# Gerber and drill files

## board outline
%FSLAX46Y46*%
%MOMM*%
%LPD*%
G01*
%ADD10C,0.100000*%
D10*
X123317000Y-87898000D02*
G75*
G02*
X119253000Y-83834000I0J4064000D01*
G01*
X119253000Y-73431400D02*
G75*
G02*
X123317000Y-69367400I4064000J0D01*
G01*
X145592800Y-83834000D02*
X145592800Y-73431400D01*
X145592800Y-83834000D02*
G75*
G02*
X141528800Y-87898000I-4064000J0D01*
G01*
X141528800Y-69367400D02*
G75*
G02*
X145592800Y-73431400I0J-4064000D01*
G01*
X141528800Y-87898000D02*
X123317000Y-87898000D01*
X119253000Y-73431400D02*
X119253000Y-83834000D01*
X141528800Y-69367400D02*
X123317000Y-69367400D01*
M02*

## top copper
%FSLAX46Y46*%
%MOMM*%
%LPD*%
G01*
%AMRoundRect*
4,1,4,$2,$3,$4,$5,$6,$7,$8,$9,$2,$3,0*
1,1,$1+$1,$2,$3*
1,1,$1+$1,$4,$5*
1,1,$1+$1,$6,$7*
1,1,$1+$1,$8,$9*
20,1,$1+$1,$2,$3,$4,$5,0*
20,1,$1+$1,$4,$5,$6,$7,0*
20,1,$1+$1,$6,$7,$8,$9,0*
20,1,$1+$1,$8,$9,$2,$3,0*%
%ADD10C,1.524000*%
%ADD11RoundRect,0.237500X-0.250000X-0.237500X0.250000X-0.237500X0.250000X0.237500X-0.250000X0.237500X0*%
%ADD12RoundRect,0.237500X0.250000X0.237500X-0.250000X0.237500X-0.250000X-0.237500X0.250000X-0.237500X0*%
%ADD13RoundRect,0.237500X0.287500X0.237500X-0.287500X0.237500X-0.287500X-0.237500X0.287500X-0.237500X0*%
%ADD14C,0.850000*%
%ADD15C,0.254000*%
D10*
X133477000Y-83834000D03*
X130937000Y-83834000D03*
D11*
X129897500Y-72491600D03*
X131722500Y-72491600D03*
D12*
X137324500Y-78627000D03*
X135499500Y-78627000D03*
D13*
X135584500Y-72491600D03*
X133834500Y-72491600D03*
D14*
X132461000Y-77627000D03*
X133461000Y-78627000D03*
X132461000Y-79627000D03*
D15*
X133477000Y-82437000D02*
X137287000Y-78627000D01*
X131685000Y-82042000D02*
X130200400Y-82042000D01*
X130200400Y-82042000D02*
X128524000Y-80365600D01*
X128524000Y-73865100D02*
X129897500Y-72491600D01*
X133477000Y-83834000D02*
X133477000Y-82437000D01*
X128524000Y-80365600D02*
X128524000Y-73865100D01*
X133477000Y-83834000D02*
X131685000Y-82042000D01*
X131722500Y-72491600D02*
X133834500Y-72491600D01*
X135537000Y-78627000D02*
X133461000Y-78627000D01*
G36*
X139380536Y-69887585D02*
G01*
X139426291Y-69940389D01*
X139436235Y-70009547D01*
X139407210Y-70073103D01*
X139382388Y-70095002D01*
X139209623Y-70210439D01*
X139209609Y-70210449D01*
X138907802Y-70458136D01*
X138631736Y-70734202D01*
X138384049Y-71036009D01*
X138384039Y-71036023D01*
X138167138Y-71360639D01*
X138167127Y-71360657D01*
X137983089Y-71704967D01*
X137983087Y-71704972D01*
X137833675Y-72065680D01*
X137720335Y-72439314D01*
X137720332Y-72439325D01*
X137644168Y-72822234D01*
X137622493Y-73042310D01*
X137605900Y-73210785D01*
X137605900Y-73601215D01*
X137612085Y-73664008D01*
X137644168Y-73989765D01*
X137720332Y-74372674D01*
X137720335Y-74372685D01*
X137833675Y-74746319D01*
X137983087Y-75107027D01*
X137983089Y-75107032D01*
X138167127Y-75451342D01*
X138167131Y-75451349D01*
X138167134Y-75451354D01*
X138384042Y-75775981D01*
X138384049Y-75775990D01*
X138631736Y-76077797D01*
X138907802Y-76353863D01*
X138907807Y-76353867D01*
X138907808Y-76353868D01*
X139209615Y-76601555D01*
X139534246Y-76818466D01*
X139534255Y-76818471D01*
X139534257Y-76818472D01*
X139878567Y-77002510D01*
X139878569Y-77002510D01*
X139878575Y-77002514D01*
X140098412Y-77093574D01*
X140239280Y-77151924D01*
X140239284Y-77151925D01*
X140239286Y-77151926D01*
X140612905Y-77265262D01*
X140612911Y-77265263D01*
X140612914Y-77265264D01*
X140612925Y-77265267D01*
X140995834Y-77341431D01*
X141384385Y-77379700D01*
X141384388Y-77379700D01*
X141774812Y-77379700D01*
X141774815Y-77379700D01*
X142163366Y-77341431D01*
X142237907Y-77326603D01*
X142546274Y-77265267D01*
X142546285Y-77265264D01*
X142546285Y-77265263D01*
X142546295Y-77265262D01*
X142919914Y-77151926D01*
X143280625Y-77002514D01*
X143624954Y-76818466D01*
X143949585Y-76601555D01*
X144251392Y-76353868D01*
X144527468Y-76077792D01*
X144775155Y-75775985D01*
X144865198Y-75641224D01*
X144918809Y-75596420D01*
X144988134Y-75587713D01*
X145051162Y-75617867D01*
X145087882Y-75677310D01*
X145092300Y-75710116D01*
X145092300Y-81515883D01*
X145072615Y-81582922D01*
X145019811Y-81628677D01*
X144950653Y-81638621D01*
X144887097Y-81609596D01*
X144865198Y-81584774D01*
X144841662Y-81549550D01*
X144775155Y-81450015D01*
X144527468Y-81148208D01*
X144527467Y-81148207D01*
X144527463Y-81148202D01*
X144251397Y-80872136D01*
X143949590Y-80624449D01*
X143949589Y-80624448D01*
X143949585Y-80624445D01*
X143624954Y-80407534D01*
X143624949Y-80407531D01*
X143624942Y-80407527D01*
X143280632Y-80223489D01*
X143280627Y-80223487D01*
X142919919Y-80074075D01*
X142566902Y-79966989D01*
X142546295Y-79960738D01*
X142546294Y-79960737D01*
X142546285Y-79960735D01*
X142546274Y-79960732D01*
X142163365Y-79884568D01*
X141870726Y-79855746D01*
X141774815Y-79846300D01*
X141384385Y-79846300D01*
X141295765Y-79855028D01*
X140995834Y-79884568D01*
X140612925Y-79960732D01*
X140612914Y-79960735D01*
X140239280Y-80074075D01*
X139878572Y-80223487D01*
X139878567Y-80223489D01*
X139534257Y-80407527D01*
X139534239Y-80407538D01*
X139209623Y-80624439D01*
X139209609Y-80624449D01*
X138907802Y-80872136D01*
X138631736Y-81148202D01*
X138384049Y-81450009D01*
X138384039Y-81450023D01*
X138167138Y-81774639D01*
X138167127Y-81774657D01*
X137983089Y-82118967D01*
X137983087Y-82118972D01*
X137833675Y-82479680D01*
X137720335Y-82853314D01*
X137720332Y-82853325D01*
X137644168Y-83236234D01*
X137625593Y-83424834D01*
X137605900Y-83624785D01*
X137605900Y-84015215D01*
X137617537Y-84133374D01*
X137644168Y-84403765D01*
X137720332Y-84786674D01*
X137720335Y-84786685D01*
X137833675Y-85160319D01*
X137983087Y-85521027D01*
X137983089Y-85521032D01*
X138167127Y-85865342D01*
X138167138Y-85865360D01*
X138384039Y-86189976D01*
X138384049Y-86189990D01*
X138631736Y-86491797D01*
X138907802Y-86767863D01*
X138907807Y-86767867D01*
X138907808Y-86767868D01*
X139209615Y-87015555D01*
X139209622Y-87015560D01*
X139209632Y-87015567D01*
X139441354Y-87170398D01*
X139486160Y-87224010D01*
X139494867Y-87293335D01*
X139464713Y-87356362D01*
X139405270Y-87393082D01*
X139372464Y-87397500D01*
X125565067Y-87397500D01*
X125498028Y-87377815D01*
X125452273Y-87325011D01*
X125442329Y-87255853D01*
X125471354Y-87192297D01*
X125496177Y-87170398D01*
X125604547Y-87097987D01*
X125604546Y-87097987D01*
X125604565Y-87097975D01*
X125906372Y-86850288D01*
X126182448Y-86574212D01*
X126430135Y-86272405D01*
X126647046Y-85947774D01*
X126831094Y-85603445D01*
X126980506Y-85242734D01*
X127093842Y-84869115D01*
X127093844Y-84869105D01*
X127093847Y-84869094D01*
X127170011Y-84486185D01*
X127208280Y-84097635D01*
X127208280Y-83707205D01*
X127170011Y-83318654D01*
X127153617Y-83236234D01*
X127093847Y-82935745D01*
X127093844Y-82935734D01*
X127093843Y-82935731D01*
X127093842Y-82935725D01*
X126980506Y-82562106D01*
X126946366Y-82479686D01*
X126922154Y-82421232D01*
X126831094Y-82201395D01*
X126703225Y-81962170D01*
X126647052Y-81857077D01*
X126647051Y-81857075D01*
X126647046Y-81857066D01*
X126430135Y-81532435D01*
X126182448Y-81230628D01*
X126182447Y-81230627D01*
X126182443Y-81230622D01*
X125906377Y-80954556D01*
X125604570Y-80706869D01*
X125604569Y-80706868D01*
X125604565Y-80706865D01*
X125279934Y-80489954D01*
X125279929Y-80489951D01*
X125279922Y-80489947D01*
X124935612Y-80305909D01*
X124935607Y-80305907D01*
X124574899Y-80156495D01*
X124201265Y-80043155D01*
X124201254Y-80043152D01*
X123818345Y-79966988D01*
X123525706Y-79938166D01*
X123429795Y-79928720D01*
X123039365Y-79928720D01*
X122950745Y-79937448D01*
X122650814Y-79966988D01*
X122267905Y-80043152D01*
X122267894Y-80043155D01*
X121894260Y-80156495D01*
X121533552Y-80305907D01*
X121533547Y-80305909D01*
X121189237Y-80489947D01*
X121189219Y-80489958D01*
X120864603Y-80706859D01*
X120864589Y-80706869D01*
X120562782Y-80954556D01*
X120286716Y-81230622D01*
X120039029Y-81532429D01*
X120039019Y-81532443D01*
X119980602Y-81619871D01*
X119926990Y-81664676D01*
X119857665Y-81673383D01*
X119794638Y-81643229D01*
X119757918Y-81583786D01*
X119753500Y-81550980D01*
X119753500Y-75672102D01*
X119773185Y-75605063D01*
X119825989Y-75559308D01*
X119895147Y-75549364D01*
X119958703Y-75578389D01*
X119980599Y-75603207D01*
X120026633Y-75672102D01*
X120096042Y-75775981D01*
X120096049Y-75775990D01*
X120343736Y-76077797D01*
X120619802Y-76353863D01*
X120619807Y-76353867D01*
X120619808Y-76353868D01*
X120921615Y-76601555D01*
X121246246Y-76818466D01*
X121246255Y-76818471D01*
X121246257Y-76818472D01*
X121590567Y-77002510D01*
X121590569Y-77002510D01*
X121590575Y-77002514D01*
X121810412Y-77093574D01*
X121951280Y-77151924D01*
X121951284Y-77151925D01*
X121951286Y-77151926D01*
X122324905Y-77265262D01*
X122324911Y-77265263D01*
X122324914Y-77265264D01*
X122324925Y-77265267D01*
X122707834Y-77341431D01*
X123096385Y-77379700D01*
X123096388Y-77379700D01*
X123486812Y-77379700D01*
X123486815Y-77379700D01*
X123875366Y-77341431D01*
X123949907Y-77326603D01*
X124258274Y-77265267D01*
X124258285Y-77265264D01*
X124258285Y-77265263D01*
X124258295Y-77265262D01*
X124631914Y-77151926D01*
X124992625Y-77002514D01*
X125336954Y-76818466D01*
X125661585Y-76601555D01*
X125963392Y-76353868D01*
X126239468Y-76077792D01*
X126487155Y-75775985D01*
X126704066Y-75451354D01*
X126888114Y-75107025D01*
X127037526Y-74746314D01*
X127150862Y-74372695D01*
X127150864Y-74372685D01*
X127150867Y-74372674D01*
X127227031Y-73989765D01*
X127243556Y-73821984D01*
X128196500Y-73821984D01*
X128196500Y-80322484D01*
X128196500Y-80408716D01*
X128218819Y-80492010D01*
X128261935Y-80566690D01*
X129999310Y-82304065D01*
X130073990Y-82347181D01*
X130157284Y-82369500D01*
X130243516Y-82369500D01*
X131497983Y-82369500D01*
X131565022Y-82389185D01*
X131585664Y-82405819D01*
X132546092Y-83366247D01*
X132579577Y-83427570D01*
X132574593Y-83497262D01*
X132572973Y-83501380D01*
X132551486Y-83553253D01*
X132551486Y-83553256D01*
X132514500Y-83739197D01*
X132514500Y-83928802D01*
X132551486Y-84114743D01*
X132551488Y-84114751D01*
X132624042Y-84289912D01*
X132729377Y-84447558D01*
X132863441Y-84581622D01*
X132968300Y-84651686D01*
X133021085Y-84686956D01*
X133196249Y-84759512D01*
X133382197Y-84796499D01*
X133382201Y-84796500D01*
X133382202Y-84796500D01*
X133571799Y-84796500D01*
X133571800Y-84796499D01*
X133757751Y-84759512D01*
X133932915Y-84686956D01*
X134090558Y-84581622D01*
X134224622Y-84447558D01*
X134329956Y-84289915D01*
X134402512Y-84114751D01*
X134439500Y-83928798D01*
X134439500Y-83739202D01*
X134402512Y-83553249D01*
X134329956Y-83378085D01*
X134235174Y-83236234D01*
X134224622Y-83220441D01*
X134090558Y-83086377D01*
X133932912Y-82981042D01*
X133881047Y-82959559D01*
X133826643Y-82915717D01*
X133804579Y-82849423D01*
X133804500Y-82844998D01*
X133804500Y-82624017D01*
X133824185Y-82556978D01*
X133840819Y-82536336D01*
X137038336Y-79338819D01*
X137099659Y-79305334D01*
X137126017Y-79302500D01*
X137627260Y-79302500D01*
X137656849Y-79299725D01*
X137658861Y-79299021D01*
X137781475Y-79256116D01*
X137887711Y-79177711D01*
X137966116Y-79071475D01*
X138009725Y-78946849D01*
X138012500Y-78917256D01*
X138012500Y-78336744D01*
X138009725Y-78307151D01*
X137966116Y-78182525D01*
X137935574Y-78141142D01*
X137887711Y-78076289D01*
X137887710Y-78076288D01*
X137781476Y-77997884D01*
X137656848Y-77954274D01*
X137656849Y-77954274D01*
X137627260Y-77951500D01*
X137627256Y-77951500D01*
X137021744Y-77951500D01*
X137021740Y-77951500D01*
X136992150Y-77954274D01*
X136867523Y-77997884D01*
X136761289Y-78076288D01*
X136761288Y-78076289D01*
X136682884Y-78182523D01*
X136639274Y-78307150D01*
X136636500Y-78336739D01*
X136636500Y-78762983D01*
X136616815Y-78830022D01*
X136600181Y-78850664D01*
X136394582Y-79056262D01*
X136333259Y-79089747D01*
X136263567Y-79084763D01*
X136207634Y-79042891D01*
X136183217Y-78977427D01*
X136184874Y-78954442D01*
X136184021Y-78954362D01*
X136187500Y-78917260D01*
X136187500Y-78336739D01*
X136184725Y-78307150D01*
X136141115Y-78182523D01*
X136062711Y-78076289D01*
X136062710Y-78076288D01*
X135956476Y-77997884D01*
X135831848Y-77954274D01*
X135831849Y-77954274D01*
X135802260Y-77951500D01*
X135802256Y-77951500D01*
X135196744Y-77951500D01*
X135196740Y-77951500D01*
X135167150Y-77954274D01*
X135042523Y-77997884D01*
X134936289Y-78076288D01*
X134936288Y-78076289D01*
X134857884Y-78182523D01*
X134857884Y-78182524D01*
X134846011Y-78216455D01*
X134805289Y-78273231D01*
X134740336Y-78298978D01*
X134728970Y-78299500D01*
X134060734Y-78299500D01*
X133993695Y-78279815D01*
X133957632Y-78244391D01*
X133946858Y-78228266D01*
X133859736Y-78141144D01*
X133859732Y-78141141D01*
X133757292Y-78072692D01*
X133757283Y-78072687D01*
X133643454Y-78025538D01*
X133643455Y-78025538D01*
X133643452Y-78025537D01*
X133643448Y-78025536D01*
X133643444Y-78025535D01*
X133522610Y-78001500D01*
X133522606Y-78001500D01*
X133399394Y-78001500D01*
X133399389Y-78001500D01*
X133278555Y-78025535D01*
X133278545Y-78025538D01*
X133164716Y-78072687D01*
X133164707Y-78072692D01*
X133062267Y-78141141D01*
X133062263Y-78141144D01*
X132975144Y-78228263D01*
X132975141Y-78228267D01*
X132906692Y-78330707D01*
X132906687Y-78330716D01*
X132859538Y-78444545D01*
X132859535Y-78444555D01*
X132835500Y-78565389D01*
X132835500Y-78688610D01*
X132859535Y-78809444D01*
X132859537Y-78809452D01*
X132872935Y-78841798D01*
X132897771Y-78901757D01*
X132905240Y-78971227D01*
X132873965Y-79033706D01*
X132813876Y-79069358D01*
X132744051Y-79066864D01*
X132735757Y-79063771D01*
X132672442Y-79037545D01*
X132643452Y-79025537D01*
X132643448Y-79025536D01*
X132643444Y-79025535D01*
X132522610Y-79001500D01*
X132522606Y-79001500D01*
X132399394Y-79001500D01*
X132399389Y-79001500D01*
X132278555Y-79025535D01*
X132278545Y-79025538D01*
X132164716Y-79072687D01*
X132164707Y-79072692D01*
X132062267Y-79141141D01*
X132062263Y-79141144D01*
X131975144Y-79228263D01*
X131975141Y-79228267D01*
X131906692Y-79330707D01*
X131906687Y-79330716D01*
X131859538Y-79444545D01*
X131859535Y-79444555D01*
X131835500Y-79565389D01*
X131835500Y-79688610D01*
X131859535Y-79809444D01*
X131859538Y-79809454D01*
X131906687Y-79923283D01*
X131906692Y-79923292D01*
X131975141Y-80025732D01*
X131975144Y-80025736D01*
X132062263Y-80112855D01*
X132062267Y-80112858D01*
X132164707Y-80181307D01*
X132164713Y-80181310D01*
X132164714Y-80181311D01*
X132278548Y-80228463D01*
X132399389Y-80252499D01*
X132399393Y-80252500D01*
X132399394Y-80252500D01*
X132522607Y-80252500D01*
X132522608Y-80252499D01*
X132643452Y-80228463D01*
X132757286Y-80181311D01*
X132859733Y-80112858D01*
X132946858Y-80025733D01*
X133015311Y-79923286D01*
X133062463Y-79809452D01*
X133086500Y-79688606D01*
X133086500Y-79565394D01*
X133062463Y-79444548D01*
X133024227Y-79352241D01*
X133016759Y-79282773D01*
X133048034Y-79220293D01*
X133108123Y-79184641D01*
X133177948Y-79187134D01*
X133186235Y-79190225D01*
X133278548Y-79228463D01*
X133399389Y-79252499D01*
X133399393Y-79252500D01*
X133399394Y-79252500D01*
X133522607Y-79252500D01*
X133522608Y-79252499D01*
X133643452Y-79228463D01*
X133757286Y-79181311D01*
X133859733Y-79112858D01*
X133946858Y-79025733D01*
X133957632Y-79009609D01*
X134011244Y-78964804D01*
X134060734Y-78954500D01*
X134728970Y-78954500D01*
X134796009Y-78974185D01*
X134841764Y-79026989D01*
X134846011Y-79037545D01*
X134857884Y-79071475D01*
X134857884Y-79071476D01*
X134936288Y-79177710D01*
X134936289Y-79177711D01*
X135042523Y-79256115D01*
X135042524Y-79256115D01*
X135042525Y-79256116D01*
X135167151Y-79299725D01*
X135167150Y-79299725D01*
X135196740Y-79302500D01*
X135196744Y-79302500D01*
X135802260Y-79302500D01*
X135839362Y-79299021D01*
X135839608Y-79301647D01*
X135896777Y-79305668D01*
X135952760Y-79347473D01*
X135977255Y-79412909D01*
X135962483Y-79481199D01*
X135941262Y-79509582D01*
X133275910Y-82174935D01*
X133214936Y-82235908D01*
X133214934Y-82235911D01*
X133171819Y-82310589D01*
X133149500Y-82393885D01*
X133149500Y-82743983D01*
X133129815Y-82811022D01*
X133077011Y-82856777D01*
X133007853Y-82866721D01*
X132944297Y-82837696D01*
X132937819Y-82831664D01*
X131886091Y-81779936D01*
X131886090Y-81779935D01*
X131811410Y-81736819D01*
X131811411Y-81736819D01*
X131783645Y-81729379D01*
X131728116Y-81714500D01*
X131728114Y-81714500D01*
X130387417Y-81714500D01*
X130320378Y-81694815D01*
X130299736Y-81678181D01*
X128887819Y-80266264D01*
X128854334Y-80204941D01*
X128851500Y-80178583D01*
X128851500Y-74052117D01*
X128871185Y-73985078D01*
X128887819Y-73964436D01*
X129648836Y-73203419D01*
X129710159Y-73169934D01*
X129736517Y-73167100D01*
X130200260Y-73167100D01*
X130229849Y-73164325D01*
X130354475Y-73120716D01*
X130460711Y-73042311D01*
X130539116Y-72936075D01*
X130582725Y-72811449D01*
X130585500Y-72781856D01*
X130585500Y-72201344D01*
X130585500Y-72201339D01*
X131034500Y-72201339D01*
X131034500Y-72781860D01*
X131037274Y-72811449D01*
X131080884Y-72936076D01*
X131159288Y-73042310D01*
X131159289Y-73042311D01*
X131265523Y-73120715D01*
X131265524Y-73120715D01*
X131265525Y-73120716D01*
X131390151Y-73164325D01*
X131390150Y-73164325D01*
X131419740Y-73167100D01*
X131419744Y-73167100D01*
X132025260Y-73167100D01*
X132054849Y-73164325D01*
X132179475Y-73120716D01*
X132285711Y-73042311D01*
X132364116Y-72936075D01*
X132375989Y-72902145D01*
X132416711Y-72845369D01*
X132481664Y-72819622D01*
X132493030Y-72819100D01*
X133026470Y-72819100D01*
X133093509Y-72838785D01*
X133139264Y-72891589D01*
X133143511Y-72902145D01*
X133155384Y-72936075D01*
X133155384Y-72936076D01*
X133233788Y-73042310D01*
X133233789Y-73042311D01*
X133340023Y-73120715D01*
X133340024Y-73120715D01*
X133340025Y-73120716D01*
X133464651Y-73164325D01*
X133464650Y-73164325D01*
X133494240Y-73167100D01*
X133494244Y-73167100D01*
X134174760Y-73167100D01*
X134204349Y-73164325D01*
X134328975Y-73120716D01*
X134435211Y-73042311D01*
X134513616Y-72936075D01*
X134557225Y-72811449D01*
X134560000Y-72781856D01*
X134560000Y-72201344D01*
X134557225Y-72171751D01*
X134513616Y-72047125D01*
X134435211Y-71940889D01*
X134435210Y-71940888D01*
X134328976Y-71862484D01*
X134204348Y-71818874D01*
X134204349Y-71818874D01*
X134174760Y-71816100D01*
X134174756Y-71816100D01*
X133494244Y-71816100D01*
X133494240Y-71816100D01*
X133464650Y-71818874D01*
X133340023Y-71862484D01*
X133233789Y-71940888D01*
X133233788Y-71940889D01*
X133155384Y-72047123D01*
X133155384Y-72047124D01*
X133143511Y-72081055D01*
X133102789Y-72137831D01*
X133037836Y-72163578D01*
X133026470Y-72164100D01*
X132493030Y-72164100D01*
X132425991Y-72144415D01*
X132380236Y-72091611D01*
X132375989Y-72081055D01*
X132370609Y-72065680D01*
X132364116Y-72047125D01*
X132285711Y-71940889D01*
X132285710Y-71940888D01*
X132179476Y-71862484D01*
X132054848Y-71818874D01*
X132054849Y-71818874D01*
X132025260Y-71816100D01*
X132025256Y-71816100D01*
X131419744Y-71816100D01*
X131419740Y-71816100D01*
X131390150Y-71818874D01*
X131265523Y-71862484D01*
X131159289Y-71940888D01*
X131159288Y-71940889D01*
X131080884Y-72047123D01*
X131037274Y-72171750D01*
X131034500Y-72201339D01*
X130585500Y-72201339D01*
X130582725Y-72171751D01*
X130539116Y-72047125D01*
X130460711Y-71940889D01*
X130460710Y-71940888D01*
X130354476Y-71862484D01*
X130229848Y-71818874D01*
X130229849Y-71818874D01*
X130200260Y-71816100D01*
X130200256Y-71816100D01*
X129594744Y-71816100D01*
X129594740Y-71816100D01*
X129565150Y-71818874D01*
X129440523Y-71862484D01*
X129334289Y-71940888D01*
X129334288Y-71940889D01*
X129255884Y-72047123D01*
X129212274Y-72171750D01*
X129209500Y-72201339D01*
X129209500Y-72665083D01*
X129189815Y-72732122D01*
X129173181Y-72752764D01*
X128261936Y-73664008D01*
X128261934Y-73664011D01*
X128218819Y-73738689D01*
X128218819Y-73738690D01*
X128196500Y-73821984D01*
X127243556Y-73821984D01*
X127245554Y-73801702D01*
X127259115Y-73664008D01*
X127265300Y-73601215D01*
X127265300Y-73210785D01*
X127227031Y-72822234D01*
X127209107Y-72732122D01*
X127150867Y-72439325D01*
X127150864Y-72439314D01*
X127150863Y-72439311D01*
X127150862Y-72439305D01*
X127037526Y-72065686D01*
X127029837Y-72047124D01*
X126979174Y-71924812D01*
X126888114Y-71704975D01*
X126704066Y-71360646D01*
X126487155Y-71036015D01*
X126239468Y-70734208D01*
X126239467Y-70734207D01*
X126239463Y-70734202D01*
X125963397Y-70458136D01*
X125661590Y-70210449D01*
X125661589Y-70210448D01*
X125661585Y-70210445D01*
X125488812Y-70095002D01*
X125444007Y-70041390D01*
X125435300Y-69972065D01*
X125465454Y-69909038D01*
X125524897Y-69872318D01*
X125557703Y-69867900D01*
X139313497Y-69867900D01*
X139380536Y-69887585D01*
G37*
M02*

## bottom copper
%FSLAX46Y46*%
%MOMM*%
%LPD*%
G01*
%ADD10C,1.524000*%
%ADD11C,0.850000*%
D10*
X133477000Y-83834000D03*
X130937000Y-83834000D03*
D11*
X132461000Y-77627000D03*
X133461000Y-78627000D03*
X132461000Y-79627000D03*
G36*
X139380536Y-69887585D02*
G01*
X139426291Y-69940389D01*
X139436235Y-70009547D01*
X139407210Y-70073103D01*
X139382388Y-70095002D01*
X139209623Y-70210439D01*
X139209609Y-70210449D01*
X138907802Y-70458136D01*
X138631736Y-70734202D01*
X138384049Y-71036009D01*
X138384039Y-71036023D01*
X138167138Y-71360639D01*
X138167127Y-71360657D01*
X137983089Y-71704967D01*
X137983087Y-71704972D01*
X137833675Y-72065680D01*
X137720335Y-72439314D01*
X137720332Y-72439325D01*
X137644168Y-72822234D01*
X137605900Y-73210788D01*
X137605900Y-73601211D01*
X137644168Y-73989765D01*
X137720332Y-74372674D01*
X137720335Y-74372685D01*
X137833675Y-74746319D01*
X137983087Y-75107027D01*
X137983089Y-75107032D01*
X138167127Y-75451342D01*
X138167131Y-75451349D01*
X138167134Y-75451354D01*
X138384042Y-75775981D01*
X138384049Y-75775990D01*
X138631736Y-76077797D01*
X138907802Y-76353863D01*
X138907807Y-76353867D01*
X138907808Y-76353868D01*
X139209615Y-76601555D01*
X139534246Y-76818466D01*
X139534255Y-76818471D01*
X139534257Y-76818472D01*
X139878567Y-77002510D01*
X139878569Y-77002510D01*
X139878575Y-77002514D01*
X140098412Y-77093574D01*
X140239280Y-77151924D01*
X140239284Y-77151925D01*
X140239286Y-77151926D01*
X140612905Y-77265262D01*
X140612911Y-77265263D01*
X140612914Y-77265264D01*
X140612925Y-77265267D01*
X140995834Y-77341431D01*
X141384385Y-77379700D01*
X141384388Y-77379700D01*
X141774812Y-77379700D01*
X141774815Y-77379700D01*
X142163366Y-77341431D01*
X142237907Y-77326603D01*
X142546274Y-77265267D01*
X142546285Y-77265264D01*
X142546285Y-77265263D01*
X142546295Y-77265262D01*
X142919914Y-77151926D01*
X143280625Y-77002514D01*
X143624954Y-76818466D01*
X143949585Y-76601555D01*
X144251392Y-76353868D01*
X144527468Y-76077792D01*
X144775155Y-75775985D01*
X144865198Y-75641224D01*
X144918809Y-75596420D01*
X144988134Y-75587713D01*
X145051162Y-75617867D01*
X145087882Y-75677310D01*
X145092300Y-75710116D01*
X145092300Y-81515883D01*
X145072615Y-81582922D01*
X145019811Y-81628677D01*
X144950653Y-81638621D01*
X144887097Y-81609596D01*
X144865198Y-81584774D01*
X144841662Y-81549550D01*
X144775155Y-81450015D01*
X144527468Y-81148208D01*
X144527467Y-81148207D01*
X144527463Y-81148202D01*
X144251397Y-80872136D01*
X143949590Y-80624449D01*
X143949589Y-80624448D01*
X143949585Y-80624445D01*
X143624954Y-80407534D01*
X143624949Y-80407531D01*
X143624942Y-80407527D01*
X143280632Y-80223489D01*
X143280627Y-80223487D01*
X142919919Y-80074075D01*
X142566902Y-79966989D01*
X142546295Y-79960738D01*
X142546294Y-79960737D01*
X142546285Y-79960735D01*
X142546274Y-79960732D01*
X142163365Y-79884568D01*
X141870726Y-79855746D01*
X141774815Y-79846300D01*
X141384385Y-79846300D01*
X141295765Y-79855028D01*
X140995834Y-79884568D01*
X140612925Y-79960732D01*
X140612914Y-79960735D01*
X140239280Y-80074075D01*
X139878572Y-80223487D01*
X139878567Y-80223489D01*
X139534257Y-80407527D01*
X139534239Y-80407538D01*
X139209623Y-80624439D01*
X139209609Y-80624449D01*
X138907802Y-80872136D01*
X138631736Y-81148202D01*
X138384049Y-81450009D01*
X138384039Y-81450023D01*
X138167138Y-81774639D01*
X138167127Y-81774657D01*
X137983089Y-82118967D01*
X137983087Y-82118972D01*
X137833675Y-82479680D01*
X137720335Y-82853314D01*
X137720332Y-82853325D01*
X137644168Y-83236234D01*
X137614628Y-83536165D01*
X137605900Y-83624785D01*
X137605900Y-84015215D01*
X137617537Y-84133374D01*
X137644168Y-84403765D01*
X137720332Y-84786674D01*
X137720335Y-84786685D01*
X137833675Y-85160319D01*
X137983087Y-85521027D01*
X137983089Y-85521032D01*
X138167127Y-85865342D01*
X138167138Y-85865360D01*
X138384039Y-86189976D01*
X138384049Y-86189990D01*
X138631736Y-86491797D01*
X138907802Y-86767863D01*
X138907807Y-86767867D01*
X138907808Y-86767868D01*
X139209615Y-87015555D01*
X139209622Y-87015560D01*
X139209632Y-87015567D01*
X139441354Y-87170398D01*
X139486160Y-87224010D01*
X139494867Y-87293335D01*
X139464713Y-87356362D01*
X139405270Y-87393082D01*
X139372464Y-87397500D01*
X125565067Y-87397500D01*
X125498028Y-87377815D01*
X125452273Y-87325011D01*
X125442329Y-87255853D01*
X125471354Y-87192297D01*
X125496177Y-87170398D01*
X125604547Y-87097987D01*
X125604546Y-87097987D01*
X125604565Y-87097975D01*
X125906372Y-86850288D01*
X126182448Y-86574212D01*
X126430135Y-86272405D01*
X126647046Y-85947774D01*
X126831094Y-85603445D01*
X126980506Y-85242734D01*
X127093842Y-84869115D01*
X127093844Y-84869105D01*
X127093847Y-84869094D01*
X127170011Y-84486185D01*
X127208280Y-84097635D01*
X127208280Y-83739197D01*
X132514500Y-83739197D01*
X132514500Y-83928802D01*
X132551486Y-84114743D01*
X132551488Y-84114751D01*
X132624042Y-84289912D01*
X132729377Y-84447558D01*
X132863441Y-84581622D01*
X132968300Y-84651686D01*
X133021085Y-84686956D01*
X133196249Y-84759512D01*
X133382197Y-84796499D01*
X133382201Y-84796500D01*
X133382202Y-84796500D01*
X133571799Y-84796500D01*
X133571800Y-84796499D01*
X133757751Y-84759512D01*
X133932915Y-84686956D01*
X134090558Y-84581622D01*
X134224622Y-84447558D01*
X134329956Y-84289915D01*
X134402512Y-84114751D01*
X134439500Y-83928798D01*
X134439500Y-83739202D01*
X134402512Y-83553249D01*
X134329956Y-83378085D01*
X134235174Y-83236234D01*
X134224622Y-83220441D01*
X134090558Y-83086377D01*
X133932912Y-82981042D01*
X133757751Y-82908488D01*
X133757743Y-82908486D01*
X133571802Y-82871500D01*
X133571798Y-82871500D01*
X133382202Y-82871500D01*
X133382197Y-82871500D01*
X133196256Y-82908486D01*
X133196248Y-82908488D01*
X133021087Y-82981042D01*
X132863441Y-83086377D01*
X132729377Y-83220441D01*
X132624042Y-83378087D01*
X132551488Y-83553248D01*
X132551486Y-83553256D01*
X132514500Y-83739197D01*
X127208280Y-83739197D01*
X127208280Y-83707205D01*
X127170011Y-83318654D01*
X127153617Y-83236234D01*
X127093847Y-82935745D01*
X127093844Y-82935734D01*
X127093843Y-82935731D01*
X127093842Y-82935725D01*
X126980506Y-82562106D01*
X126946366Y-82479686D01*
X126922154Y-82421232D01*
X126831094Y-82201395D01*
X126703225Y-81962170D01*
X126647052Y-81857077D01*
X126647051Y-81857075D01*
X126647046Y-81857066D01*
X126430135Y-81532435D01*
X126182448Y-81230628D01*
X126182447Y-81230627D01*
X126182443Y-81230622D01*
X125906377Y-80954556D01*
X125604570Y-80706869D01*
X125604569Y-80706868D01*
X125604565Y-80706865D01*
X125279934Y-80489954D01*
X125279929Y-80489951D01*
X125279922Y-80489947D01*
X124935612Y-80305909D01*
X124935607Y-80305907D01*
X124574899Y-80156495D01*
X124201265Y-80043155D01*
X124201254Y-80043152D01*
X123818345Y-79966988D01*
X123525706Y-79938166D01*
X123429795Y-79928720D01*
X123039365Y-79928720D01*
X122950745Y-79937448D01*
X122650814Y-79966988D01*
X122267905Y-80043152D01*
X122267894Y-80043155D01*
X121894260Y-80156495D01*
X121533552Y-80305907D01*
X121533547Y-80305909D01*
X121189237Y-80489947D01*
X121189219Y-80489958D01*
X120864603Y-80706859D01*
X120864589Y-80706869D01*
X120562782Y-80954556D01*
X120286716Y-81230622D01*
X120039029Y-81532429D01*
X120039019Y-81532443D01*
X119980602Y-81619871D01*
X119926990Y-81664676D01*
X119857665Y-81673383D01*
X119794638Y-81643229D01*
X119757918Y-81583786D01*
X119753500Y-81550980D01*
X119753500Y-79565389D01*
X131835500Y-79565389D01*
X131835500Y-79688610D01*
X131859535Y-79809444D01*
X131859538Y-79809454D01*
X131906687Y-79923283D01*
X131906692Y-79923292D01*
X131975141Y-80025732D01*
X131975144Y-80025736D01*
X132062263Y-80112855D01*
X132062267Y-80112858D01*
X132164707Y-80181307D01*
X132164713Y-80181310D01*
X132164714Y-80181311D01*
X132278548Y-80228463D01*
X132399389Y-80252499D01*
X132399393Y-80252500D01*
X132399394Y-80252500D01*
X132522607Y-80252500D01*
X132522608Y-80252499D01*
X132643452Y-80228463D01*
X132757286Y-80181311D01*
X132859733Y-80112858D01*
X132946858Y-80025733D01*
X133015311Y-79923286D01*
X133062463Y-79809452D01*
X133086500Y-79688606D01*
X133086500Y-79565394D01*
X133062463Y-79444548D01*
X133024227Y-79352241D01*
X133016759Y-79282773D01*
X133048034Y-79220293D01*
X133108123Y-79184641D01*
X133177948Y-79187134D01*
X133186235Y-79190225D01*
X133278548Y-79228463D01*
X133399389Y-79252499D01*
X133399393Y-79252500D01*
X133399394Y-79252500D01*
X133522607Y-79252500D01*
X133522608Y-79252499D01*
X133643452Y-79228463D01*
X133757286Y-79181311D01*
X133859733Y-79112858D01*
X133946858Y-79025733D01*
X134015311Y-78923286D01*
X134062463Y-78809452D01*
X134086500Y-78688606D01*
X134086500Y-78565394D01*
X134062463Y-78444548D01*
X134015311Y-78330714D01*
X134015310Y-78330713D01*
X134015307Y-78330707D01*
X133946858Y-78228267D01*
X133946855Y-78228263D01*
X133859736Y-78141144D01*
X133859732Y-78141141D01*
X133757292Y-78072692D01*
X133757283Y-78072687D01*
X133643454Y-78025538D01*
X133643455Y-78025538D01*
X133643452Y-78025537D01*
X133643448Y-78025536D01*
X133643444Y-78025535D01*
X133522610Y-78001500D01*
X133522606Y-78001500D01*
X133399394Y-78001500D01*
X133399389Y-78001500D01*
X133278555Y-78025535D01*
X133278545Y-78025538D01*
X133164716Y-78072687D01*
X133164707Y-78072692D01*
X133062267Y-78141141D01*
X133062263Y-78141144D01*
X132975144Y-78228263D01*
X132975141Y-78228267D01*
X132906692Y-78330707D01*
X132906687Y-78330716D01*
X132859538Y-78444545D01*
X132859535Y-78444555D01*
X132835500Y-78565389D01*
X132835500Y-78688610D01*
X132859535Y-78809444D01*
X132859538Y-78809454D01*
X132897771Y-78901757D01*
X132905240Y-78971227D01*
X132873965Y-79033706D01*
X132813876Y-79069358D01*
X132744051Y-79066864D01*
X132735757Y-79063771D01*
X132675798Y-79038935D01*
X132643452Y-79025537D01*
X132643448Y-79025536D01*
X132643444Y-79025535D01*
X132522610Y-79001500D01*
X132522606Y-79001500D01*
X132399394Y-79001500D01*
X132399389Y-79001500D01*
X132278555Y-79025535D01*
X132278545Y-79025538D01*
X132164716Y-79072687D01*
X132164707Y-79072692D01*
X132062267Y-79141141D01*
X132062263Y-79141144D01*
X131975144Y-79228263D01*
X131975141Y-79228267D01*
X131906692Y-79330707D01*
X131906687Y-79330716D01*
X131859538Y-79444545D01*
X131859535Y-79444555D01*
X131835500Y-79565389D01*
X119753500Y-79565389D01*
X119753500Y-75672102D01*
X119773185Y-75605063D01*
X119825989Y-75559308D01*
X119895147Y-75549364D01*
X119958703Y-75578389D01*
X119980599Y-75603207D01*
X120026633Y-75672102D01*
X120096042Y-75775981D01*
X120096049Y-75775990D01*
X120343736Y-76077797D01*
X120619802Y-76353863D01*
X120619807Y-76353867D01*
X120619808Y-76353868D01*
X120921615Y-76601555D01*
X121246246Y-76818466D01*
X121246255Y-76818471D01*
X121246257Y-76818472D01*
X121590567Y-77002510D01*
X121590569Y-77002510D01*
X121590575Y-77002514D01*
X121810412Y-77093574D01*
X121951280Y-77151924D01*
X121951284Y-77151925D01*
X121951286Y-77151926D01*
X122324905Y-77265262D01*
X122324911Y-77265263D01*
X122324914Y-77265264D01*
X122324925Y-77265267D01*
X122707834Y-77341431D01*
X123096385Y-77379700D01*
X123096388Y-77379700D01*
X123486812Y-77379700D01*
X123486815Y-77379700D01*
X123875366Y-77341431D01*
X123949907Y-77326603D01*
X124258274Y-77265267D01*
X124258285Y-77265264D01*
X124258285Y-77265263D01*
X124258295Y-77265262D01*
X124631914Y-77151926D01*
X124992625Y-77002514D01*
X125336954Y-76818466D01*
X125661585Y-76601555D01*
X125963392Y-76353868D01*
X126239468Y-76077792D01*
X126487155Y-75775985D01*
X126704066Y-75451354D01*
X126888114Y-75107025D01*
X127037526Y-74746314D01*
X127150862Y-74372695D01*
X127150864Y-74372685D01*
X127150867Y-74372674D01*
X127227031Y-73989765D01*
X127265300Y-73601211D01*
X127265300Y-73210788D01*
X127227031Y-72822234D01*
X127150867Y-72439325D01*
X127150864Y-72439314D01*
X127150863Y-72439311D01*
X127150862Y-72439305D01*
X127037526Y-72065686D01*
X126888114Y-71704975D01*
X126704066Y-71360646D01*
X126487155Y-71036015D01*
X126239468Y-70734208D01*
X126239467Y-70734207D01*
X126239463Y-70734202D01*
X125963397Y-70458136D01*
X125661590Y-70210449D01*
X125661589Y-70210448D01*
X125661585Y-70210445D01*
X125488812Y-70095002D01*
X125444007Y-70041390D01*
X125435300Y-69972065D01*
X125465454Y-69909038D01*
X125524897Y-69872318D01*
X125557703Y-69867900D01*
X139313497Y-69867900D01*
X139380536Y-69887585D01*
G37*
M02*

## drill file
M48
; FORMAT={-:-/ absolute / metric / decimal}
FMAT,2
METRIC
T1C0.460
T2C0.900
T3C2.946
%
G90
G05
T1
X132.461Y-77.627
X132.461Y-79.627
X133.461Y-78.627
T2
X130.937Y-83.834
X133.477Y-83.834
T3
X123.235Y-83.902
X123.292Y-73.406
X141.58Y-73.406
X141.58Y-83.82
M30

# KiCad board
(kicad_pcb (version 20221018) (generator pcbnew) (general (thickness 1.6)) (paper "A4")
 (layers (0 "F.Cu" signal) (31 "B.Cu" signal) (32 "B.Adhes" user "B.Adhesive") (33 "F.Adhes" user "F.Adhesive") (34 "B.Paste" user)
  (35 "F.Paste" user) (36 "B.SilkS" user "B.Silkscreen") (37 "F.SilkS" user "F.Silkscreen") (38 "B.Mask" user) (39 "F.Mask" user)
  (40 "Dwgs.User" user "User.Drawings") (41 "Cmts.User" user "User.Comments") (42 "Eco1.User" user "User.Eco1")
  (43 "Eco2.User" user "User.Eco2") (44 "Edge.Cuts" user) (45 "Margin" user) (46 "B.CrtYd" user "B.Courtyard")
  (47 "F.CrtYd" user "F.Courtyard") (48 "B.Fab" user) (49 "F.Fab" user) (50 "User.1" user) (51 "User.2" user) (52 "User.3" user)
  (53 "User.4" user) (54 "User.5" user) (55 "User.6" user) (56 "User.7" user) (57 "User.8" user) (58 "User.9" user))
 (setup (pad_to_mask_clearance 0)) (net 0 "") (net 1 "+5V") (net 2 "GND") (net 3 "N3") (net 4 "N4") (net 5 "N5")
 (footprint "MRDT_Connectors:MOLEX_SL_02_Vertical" (layer "F.Cu") (at 133.477 83.834 180)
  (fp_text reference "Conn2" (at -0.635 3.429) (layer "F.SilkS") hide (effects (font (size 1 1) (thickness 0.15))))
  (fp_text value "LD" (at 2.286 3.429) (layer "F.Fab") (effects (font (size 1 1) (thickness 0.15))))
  (pad "1" thru_hole circle (at 0 0 180) (size 1.524 1.524) (drill 0.9) (layers "*.Cu" "*.Mask") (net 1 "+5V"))
  (pad "2" thru_hole circle (at 2.54 0 180) (size 1.524 1.524) (drill 0.9) (layers "*.Cu" "*.Mask") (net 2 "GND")))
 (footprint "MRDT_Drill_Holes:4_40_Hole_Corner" (layer "F.Cu") (at 127.2427 79.8943 180)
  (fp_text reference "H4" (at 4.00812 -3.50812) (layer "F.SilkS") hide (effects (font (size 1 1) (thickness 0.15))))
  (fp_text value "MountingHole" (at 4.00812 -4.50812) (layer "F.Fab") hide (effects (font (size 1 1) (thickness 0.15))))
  (pad "" np_thru_hole circle (at 4.00812 -4.00812 180) (size 2.9464 2.9464) (drill 2.9464) (layers "*.Cu" "*.Mask") (clearance 2.5)))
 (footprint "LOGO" (layer "F.Cu") (at 128.27 77.089)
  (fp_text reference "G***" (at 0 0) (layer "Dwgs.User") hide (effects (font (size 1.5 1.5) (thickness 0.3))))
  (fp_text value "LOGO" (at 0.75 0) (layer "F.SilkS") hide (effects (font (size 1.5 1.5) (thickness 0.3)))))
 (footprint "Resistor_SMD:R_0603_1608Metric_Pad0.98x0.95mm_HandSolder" (layer "F.Cu") (at 130.81 72.4916)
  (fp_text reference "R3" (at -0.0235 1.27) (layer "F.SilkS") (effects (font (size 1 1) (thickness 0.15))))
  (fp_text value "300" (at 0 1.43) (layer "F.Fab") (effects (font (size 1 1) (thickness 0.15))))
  (pad "1" smd roundrect (at -0.9125 0) (size 0.975 0.95) (layers "F.Cu" "F.Paste" "F.Mask") (roundrect_rratio 0.25) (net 1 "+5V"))
  (pad "2" smd roundrect (at 0.9125 0) (size 0.975 0.95) (layers "F.Cu" "F.Paste" "F.Mask") (roundrect_rratio 0.25) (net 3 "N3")))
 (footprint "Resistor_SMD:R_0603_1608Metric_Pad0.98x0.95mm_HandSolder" (layer "F.Cu") (at 136.412 78.627 180)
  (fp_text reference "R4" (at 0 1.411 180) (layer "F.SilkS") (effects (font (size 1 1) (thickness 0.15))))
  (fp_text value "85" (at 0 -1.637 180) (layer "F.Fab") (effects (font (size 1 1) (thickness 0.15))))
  (pad "1" smd roundrect (at -0.9125 0 180) (size 0.975 0.95) (layers "F.Cu" "F.Paste" "F.Mask") (roundrect_rratio 0.25) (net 1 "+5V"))
  (pad "2" smd roundrect (at 0.9125 0 180) (size 0.975 0.95) (layers "F.Cu" "F.Paste" "F.Mask") (roundrect_rratio 0.25) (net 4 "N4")))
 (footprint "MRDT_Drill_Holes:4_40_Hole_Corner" (layer "F.Cu") (at 127.29972 77.41412 90)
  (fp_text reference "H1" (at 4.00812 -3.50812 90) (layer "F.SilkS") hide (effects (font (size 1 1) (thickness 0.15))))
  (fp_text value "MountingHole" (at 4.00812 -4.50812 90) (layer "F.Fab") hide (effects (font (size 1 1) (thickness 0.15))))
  (pad "" np_thru_hole circle (at 4.00812 -4.00812 90) (size 2.9464 2.9464) (drill 2.9464) (layers "*.Cu" "*.Mask") (clearance 2.5)))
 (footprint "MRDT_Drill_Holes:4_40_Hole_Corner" (layer "F.Cu") (at 137.57148 79.81188 -90)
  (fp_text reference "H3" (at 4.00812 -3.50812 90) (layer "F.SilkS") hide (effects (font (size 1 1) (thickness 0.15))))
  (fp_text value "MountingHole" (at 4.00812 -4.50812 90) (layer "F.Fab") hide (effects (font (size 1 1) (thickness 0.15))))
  (pad "" np_thru_hole circle (at 4.00812 -4.00812 270) (size 2.9464 2.9464) (drill 2.9464) (layers "*.Cu" "*.Mask") (clearance 2.5)))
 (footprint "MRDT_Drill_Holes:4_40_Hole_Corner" (layer "F.Cu") (at 137.57148 77.41412)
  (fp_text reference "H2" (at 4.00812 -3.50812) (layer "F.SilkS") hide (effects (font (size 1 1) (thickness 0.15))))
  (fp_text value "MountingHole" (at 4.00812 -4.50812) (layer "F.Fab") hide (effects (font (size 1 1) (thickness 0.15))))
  (pad "" np_thru_hole circle (at 4.00812 -4.00812) (size 2.9464 2.9464) (drill 2.9464) (layers "*.Cu" "*.Mask") (clearance 2.5)))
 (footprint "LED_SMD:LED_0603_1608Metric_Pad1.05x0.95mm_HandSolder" (layer "F.Cu") (at 134.7095 72.4916 180)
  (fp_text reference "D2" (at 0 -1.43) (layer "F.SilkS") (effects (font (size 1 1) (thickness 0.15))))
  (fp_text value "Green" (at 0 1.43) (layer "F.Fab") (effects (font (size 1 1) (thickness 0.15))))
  (pad "1" smd roundrect (at -0.875 0 180) (size 1.05 0.95) (layers "F.Cu" "F.Paste" "F.Mask") (roundrect_rratio 0.25) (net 2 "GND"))
  (pad "2" smd roundrect (at 0.875 0 180) (size 1.05 0.95) (layers "F.Cu" "F.Paste" "F.Mask") (roundrect_rratio 0.25) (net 3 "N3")))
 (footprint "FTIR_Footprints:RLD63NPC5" (layer "B.Cu") (at 132.461 78.627 180)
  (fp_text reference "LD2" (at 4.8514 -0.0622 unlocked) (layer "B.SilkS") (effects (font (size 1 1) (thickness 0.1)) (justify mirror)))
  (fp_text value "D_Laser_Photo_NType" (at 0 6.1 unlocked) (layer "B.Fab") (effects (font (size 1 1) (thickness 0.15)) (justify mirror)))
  (pad "1" thru_hole circle (at 0 1 180) (size 0.85 0.85) (drill 0.46) (layers "*.Cu" "*.Mask") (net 2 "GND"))
  (pad "2" thru_hole circle (at -1 0 180) (size 0.85 0.85) (drill 0.46) (layers "*.Cu" "*.Mask") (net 4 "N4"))
  (pad "3" thru_hole circle (at 0 -1 180) (size 0.85 0.85) (drill 0.46) (layers "*.Cu" "*.Mask") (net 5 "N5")))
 (gr_arc (start 123.317 87.898) (mid 120.443318 86.707682) (end 119.253 83.834) (stroke (width 0.1) (type default)) (layer "Edge.Cuts"))
 (gr_arc (start 119.253 73.4314) (mid 120.443318 70.557718) (end 123.317 69.3674) (stroke (width 0.1) (type default)) (layer "Edge.Cuts"))
 (gr_line (start 145.5928 83.834) (end 145.5928 73.4314) (stroke (width 0.1) (type default)) (layer "Edge.Cuts"))
 (gr_arc (start 145.5928 83.834) (mid 144.402482 86.707682) (end 141.5288 87.898) (stroke (width 0.1) (type default)) (layer "Edge.Cuts"))
 (gr_arc (start 141.5288 69.3674) (mid 144.402482 70.557718) (end 145.5928 73.4314) (stroke (width 0.1) (type default)) (layer "Edge.Cuts"))
 (gr_line (start 141.5288 87.898) (end 123.317 87.898) (stroke (width 0.1) (type default)) (layer "Edge.Cuts"))
 (gr_line (start 119.253 73.4314) (end 119.253 83.834) (stroke (width 0.1) (type default)) (layer "Edge.Cuts"))
 (gr_line (start 141.5288 69.3674) (end 123.317 69.3674) (stroke (width 0.1) (type default)) (layer "Edge.Cuts"))
 (segment (start 133.477 82.437) (end 137.287 78.627) (width 0.254) (layer "F.Cu") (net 1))
 (segment (start 131.685 82.042) (end 130.2004 82.042) (width 0.254) (layer "F.Cu") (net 1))
 (segment (start 130.2004 82.042) (end 128.524 80.3656) (width 0.254) (layer "F.Cu") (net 1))
 (segment (start 128.524 73.8651) (end 129.8975 72.4916) (width 0.254) (layer "F.Cu") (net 1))
 (segment (start 133.477 83.834) (end 133.477 82.437) (width 0.254) (layer "F.Cu") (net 1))
 (segment (start 128.524 80.3656) (end 128.524 73.8651) (width 0.254) (layer "F.Cu") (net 1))
 (segment (start 133.477 83.834) (end 131.685 82.042) (width 0.254) (layer "F.Cu") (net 1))
 (segment (start 131.7225 72.4916) (end 133.8345 72.4916) (width 0.254) (layer "F.Cu") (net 3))
 (segment (start 135.537 78.627) (end 133.461 78.627) (width 0.254) (layer "F.Cu") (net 4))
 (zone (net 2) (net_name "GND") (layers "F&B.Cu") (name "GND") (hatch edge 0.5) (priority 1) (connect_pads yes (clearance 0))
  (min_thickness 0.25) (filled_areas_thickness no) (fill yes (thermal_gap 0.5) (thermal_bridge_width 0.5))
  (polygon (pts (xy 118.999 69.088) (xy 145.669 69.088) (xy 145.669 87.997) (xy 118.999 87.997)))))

